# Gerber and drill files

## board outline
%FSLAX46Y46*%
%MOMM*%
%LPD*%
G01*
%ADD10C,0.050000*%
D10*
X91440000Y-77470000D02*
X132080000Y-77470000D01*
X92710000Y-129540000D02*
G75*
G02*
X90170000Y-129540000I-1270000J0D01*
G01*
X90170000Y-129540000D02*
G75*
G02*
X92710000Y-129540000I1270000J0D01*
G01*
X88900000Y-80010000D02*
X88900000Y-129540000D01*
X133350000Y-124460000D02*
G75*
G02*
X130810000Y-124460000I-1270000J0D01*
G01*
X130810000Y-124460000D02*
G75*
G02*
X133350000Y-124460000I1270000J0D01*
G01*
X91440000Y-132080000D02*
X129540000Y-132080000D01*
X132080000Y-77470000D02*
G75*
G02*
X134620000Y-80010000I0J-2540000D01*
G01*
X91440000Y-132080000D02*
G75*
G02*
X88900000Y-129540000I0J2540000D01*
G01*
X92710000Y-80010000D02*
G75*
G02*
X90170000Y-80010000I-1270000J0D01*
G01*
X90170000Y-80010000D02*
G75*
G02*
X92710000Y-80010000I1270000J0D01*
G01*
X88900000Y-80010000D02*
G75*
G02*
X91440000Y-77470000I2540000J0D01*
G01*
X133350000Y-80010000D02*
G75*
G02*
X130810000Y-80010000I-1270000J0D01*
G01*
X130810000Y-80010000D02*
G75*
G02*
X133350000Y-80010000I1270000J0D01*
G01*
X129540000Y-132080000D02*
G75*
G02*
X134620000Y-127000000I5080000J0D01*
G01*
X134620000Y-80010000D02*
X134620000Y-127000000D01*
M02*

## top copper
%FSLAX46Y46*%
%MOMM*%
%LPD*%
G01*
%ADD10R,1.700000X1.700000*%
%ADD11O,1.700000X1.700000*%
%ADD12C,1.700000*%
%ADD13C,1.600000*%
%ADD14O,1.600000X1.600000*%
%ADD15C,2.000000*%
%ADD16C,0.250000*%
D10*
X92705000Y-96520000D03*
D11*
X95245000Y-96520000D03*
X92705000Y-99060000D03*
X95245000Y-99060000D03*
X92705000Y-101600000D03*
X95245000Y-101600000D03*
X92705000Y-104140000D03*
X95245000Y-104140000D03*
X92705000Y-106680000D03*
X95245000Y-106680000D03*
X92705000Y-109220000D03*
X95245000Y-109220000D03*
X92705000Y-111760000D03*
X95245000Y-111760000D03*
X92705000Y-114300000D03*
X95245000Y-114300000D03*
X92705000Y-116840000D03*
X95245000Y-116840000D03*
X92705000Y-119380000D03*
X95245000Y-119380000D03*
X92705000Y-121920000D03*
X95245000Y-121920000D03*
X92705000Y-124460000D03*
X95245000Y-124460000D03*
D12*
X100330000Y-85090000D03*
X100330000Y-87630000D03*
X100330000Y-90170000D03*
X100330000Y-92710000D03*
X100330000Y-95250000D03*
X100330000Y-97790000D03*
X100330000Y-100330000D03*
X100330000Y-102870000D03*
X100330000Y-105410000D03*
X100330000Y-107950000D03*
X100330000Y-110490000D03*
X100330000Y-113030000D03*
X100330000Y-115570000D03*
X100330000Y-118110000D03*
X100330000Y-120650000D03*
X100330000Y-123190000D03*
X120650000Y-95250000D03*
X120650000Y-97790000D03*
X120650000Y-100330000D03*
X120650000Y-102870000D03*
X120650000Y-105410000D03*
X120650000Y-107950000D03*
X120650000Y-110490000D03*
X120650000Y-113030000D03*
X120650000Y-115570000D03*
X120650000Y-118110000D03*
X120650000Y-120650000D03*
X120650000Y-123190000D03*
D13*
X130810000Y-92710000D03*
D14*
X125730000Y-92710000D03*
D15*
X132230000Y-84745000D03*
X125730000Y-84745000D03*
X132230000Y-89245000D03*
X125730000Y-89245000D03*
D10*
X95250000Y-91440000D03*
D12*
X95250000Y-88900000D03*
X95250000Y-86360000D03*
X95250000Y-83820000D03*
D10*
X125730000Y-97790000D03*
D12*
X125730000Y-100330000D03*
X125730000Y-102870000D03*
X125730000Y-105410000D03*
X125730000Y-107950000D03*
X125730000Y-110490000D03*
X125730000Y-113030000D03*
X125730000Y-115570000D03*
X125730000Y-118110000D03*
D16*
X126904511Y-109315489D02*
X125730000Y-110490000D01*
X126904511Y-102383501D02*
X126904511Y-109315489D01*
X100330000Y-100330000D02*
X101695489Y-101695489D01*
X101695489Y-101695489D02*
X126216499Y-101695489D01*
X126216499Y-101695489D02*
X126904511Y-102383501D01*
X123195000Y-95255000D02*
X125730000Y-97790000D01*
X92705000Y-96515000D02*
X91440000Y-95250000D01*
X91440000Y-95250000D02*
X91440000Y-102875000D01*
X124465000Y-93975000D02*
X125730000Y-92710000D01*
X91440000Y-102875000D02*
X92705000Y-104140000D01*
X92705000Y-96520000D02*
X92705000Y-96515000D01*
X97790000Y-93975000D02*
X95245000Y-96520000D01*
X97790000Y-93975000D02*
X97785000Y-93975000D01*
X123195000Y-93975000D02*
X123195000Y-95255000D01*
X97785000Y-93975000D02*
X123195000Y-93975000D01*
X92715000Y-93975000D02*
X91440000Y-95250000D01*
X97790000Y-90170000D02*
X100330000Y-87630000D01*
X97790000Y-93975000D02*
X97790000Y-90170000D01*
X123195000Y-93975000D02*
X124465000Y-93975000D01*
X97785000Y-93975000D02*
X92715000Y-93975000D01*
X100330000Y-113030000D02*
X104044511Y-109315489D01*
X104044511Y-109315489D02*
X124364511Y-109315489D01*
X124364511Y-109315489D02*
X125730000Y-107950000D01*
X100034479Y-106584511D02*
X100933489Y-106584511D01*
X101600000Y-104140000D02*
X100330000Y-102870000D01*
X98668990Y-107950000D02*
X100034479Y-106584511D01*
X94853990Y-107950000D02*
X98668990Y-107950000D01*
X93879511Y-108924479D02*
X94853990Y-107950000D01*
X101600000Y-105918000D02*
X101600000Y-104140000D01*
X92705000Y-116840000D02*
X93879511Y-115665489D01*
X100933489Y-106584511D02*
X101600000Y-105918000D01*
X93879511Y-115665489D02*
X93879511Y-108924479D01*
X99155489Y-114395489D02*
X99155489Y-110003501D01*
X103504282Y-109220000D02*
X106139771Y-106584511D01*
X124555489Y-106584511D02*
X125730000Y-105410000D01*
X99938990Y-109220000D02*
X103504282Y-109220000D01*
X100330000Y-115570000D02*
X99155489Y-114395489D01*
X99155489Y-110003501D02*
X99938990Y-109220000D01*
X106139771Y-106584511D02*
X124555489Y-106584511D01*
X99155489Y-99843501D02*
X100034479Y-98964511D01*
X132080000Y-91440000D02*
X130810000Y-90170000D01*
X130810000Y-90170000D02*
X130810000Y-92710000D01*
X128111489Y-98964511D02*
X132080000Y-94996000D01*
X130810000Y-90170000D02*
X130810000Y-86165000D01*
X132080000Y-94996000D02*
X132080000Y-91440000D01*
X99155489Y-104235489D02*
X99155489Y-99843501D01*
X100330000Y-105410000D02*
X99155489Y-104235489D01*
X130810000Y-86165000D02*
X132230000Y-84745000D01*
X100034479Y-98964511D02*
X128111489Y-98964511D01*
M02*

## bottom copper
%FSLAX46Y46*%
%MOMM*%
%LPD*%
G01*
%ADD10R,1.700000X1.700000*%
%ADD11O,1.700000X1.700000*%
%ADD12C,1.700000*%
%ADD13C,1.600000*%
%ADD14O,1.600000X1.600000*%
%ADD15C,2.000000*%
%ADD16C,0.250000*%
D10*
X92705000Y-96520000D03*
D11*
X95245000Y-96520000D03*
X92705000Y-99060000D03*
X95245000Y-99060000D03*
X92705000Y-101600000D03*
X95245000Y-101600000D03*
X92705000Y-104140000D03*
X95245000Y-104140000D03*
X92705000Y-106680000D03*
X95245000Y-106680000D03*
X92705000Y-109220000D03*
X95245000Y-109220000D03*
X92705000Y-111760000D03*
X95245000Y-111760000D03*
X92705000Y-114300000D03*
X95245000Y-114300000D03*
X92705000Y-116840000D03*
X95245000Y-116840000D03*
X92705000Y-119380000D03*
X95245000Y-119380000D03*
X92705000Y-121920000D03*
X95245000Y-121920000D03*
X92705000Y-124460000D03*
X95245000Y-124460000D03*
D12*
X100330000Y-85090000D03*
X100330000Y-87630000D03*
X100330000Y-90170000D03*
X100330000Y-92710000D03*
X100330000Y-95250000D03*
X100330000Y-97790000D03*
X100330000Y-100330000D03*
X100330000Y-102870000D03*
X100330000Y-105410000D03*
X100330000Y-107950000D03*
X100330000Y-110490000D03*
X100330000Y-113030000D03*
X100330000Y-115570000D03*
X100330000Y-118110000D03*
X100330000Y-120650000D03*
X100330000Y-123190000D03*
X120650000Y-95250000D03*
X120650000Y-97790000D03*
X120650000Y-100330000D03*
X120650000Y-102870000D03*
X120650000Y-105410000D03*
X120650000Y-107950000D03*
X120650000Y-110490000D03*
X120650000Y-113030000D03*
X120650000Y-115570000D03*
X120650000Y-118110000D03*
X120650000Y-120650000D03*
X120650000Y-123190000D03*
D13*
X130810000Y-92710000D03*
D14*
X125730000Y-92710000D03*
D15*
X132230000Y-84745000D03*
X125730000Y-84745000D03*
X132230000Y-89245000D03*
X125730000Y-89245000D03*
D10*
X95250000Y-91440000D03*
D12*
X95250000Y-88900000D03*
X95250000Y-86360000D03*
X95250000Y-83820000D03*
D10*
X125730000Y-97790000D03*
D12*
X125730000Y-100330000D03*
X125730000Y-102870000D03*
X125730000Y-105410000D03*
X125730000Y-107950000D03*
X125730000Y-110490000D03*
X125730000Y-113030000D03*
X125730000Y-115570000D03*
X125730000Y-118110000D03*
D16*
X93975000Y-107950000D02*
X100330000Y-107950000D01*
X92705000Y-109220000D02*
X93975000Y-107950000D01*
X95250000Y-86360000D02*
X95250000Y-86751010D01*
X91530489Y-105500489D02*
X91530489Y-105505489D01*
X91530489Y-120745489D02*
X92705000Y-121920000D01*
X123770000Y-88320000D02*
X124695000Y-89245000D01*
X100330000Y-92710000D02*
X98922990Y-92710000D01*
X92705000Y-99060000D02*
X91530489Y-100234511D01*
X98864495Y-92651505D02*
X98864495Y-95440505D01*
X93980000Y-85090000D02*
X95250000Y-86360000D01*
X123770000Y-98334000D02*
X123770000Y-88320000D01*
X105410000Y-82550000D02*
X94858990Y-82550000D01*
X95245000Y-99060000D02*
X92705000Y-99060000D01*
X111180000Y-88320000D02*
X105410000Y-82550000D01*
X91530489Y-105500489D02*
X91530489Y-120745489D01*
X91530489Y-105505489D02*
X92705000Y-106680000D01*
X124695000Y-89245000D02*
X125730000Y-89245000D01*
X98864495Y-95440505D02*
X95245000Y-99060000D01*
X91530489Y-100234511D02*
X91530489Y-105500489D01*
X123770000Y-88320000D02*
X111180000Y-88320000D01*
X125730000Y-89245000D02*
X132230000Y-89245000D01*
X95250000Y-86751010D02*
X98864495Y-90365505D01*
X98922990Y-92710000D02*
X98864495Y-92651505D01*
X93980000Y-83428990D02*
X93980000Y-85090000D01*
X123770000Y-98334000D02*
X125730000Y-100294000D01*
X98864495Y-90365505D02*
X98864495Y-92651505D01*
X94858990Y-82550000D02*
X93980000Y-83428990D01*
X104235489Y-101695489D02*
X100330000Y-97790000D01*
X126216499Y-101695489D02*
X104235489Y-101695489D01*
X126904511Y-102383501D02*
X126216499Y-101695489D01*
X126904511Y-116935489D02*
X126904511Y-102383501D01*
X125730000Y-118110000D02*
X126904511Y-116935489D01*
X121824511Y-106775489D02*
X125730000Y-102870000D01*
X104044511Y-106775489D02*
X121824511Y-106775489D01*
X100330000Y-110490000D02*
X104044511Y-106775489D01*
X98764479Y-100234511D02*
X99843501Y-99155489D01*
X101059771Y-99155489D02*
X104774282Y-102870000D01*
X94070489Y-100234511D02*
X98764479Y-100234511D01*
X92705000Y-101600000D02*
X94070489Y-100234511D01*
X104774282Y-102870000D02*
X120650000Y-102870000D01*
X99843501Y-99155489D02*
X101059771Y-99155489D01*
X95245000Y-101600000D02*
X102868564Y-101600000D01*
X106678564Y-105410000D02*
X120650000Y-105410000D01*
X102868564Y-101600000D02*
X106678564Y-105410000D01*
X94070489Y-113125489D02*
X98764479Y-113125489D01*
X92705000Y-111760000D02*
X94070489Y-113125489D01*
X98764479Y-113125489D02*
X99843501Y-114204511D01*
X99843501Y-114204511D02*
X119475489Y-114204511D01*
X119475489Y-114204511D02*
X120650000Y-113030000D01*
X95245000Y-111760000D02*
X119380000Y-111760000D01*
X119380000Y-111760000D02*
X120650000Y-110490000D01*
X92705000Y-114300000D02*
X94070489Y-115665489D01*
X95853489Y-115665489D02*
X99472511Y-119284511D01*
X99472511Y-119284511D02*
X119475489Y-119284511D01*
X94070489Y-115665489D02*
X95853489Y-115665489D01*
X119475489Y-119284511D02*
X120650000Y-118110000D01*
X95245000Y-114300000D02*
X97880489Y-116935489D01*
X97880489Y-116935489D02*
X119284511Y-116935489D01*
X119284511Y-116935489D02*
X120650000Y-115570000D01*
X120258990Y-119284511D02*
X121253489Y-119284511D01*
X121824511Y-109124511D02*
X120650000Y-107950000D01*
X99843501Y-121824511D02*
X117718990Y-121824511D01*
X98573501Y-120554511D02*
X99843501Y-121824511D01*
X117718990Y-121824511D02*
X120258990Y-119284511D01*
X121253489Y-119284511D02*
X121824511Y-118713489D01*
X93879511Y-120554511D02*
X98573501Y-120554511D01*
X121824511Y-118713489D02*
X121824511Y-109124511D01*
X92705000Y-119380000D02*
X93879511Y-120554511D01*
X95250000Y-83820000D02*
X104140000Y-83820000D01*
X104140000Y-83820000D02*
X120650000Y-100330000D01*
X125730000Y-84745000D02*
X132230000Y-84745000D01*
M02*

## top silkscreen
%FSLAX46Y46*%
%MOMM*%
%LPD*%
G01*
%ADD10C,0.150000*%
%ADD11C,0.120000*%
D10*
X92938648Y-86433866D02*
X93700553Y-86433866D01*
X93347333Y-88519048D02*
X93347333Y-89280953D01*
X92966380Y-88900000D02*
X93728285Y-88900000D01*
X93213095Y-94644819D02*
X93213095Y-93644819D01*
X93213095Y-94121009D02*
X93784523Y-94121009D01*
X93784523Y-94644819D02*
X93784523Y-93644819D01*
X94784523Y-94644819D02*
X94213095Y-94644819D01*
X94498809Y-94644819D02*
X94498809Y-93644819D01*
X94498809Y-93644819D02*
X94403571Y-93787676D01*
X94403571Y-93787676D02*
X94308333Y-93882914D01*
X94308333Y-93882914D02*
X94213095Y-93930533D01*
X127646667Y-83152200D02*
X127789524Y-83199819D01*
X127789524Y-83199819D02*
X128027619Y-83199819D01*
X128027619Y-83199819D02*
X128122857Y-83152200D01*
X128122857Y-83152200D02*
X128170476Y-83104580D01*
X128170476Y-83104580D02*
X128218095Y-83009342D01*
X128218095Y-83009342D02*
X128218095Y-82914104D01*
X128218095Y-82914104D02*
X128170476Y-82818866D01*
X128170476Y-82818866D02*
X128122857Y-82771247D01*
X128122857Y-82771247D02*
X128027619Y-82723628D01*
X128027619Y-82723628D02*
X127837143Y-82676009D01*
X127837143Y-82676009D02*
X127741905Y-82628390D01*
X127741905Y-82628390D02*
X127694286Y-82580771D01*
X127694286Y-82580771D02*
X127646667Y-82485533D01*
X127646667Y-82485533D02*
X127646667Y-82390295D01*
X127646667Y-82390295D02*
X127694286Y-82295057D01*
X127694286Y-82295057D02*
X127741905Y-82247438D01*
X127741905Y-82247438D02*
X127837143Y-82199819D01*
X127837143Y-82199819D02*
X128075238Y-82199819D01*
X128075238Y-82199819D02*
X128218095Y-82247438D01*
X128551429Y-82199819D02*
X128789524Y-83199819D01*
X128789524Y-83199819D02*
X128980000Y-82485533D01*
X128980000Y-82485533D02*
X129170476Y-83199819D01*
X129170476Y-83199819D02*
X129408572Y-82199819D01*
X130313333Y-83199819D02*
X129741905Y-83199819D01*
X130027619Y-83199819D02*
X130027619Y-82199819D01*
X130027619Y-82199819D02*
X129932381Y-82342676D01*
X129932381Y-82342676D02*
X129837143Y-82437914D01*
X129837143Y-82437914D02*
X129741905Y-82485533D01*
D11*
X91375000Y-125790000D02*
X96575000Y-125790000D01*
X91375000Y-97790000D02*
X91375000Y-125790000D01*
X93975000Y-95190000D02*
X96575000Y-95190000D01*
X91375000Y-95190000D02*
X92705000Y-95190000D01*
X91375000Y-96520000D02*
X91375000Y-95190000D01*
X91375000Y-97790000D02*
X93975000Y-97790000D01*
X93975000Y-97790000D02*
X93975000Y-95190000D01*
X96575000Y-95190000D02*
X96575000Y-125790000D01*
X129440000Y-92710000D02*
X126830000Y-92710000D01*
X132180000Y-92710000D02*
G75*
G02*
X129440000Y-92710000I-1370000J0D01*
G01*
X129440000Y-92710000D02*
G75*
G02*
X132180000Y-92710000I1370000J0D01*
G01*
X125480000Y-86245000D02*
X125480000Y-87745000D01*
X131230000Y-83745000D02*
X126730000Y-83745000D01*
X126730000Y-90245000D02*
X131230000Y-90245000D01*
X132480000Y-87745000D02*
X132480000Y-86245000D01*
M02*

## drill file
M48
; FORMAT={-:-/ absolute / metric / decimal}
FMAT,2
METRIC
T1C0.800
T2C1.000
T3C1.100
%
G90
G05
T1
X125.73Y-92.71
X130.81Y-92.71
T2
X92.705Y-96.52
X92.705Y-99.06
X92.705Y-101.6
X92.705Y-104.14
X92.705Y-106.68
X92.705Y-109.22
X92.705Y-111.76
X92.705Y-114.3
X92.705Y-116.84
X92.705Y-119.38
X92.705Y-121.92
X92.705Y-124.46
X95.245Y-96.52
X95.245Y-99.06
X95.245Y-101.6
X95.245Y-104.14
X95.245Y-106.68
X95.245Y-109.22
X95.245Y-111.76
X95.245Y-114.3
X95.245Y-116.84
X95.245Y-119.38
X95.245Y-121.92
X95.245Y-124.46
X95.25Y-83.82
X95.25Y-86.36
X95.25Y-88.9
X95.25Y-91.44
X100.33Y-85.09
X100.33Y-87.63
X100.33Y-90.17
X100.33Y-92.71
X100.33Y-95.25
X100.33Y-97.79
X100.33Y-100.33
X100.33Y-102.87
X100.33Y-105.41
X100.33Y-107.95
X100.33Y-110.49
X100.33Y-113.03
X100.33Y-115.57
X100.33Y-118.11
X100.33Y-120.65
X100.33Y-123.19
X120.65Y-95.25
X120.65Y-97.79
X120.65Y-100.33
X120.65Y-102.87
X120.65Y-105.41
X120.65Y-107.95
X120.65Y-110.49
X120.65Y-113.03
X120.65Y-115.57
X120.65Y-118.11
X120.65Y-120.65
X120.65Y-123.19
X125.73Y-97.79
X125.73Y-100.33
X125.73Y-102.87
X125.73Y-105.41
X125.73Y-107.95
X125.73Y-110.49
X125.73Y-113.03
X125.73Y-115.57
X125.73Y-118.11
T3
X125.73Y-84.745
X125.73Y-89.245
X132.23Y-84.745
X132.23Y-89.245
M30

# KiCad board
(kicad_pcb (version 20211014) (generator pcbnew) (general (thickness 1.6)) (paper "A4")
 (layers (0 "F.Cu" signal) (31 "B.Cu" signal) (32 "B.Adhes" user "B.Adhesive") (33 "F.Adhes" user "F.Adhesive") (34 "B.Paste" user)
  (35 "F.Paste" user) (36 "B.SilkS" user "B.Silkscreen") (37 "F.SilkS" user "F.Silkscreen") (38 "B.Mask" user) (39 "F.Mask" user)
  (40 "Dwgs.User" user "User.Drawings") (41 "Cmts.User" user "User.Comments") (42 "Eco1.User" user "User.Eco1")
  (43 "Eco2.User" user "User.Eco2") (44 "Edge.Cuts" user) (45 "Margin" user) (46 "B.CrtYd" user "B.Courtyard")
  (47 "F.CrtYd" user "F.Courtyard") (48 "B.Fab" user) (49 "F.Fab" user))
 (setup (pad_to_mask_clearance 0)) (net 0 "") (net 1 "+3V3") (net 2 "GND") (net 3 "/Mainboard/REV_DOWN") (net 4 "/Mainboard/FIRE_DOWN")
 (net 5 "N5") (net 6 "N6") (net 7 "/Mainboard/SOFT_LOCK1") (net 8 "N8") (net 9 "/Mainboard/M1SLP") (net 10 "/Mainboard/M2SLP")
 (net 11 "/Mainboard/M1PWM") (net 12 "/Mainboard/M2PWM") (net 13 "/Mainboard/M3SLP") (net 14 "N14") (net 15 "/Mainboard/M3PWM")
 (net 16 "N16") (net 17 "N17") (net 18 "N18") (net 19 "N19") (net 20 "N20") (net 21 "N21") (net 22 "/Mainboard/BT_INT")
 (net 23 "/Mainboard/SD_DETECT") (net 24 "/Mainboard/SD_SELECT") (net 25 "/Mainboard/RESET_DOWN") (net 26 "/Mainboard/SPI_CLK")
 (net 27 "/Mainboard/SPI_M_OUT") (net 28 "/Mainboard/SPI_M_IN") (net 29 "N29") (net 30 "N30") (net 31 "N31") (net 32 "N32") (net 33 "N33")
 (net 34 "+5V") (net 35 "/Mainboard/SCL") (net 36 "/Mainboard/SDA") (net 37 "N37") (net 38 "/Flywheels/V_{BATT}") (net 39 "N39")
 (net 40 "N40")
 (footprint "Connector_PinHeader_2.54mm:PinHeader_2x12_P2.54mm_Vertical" (layer "F.Cu") (at 92.705 96.52)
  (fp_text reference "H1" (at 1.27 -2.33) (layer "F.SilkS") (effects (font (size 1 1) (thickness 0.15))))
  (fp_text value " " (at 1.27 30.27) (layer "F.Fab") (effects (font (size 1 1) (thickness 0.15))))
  (fp_line (start -1.33 29.27) (end 3.87 29.27) (layer "F.SilkS") (width 0.12))
  (fp_line (start -1.33 1.27) (end -1.33 29.27) (layer "F.SilkS") (width 0.12))
  (fp_line (start 1.27 -1.33) (end 3.87 -1.33) (layer "F.SilkS") (width 0.12))
  (fp_line (start -1.33 -1.33) (end 0 -1.33) (layer "F.SilkS") (width 0.12))
  (fp_line (start -1.33 0) (end -1.33 -1.33) (layer "F.SilkS") (width 0.12))
  (fp_line (start -1.33 1.27) (end 1.27 1.27) (layer "F.SilkS") (width 0.12))
  (fp_line (start 1.27 1.27) (end 1.27 -1.33) (layer "F.SilkS") (width 0.12))
  (fp_line (start 3.87 -1.33) (end 3.87 29.27) (layer "F.SilkS") (width 0.12))
  (pad "1" thru_hole rect locked (at 0 0) (size 1.7 1.7) (drill 1) (layers *.Cu *.Mask) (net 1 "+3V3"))
  (pad "2" thru_hole oval locked (at 2.54 0) (size 1.7 1.7) (drill 1) (layers *.Cu *.Mask) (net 1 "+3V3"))
  (pad "3" thru_hole oval locked (at 0 2.54) (size 1.7 1.7) (drill 1) (layers *.Cu *.Mask) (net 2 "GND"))
  (pad "4" thru_hole oval locked (at 2.54 2.54) (size 1.7 1.7) (drill 1) (layers *.Cu *.Mask) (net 2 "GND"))
  (pad "5" thru_hole oval locked (at 0 5.08) (size 1.7 1.7) (drill 1) (layers *.Cu *.Mask) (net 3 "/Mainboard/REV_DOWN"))
  (pad "6" thru_hole oval locked (at 2.54 5.08) (size 1.7 1.7) (drill 1) (layers *.Cu *.Mask) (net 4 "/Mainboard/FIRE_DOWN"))
  (pad "7" thru_hole oval locked (at 0 7.62) (size 1.7 1.7) (drill 1) (layers *.Cu *.Mask) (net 1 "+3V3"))
  (pad "8" thru_hole oval locked (at 2.54 7.62) (size 1.7 1.7) (drill 1) (layers *.Cu *.Mask) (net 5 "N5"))
  (pad "9" thru_hole oval locked (at 0 10.16) (size 1.7 1.7) (drill 1) (layers *.Cu *.Mask) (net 2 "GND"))
  (pad "10" thru_hole oval locked (at 2.54 10.16) (size 1.7 1.7) (drill 1) (layers *.Cu *.Mask) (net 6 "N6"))
  (pad "11" thru_hole oval locked (at 0 12.7) (size 1.7 1.7) (drill 1) (layers *.Cu *.Mask) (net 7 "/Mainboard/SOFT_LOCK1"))
  (pad "12" thru_hole oval locked (at 2.54 12.7) (size 1.7 1.7) (drill 1) (layers *.Cu *.Mask) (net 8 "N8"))
  (pad "13" thru_hole oval locked (at 0 15.24) (size 1.7 1.7) (drill 1) (layers *.Cu *.Mask) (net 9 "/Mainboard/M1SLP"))
  (pad "14" thru_hole oval locked (at 2.54 15.24) (size 1.7 1.7) (drill 1) (layers *.Cu *.Mask) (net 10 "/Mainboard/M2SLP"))
  (pad "15" thru_hole oval locked (at 0 17.78) (size 1.7 1.7) (drill 1) (layers *.Cu *.Mask) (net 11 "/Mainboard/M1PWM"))
  (pad "16" thru_hole oval locked (at 2.54 17.78) (size 1.7 1.7) (drill 1) (layers *.Cu *.Mask) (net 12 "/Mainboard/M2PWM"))
  (pad "17" thru_hole oval locked (at 0 20.32) (size 1.7 1.7) (drill 1) (layers *.Cu *.Mask) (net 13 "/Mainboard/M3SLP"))
  (pad "18" thru_hole oval locked (at 2.54 20.32) (size 1.7 1.7) (drill 1) (layers *.Cu *.Mask) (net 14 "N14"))
  (pad "19" thru_hole oval locked (at 0 22.86) (size 1.7 1.7) (drill 1) (layers *.Cu *.Mask) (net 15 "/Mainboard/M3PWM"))
  (pad "20" thru_hole oval locked (at 2.54 22.86) (size 1.7 1.7) (drill 1) (layers *.Cu *.Mask) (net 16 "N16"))
  (pad "21" thru_hole oval locked (at 0 25.4) (size 1.7 1.7) (drill 1) (layers *.Cu *.Mask) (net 2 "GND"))
  (pad "22" thru_hole oval locked (at 2.54 25.4) (size 1.7 1.7) (drill 1) (layers *.Cu *.Mask) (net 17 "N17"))
  (pad "23" thru_hole oval locked (at 0 27.94) (size 1.7 1.7) (drill 1) (layers *.Cu *.Mask) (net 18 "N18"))
  (pad "24" thru_hole oval locked (at 2.54 27.94) (size 1.7 1.7) (drill 1) (layers *.Cu *.Mask) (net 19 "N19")))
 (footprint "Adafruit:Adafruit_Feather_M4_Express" (layer "F.Cu") (at 110.49 104.14)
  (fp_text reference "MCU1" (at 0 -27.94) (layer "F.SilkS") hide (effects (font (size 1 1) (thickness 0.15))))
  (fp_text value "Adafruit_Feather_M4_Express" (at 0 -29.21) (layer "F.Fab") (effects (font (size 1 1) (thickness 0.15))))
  (pad "1" thru_hole circle (at -10.16 -19.05) (size 1.7 1.7) (drill 1) (layers *.Cu *.Mask) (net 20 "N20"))
  (pad "2" thru_hole circle (at -10.16 -16.51) (size 1.7 1.7) (drill 1) (layers *.Cu *.Mask) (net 1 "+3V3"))
  (pad "3" thru_hole circle (at -10.16 -13.97) (size 1.7 1.7) (drill 1) (layers *.Cu *.Mask) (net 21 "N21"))
  (pad "4" thru_hole circle (at -10.16 -11.43) (size 1.7 1.7) (drill 1) (layers *.Cu *.Mask) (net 2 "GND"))
  (pad "5" thru_hole circle (at -10.16 -8.89) (size 1.7 1.7) (drill 1) (layers *.Cu *.Mask) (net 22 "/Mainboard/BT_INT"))
  (pad "6" thru_hole circle (at -10.16 -6.35) (size 1.7 1.7) (drill 1) (layers *.Cu *.Mask) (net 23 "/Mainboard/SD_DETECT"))
  (pad "7" thru_hole circle (at -10.16 -3.81) (size 1.7 1.7) (drill 1) (layers *.Cu *.Mask) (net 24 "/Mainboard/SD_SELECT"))
  (pad "8" thru_hole circle (at -10.16 -1.27) (size 1.7 1.7) (drill 1) (layers *.Cu *.Mask) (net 13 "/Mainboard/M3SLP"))
  (pad "9" thru_hole circle (at -10.16 1.27) (size 1.7 1.7) (drill 1) (layers *.Cu *.Mask) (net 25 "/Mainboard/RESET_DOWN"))
  (pad "10" thru_hole circle (at -10.16 3.81) (size 1.7 1.7) (drill 1) (layers *.Cu *.Mask) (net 7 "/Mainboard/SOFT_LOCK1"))
  (pad "11" thru_hole circle (at -10.16 6.35) (size 1.7 1.7) (drill 1) (layers *.Cu *.Mask) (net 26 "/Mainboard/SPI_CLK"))
  (pad "12" thru_hole circle (at -10.16 8.89) (size 1.7 1.7) (drill 1) (layers *.Cu *.Mask) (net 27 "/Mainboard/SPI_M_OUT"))
  (pad "13" thru_hole circle (at -10.16 11.43) (size 1.7 1.7) (drill 1) (layers *.Cu *.Mask) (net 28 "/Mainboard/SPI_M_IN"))
  (pad "14" thru_hole circle (at -10.16 13.97) (size 1.7 1.7) (drill 1) (layers *.Cu *.Mask) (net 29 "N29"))
  (pad "15" thru_hole circle (at -10.16 16.51) (size 1.7 1.7) (drill 1) (layers *.Cu *.Mask) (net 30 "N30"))
  (pad "16" thru_hole circle (at -10.16 19.05) (size 1.7 1.7) (drill 1) (layers *.Cu *.Mask) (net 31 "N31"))
  (pad "17" thru_hole circle (at 10.16 -8.89) (size 1.7 1.7) (drill 1) (layers *.Cu *.Mask) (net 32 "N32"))
  (pad "18" thru_hole circle (at 10.16 -6.35) (size 1.7 1.7) (drill 1) (layers *.Cu *.Mask) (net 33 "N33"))
  (pad "19" thru_hole circle (at 10.16 -3.81) (size 1.7 1.7) (drill 1) (layers *.Cu *.Mask) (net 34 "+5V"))
  (pad "20" thru_hole circle (at 10.16 -1.27) (size 1.7 1.7) (drill 1) (layers *.Cu *.Mask) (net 3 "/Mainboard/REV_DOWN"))
  (pad "21" thru_hole circle (at 10.16 1.27) (size 1.7 1.7) (drill 1) (layers *.Cu *.Mask) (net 4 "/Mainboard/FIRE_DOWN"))
  (pad "22" thru_hole circle (at 10.16 3.81) (size 1.7 1.7) (drill 1) (layers *.Cu *.Mask) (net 15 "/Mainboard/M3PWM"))
  (pad "23" thru_hole circle (at 10.16 6.35) (size 1.7 1.7) (drill 1) (layers *.Cu *.Mask) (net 10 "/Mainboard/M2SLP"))
  (pad "24" thru_hole circle (at 10.16 8.89) (size 1.7 1.7) (drill 1) (layers *.Cu *.Mask) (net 9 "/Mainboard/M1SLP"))
  (pad "25" thru_hole circle (at 10.16 11.43) (size 1.7 1.7) (drill 1) (layers *.Cu *.Mask) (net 12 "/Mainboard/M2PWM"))
  (pad "26" thru_hole circle (at 10.16 13.97) (size 1.7 1.7) (drill 1) (layers *.Cu *.Mask) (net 11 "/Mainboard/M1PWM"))
  (pad "27" thru_hole circle (at 10.16 16.51) (size 1.7 1.7) (drill 1) (layers *.Cu *.Mask) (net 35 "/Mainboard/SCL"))
  (pad "28" thru_hole circle (at 10.16 19.05) (size 1.7 1.7) (drill 1) (layers *.Cu *.Mask) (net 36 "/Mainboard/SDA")))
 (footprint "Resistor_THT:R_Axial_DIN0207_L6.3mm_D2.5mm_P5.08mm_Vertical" (layer "F.Cu") (at 130.81 92.71 180)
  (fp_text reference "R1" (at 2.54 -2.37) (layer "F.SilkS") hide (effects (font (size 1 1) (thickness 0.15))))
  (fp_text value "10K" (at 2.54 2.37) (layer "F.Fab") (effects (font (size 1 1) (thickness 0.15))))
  (fp_line (start 1.37 0) (end 3.98 0) (layer "F.SilkS") (width 0.12))
  (fp_circle (center 0 0) (end 1.37 0) (layer "F.SilkS") (width 0.12) (fill none))
  (pad "1" thru_hole circle locked (at 0 0 180) (size 1.6 1.6) (drill 0.8) (layers *.Cu *.Mask) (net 25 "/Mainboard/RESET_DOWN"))
  (pad "2" thru_hole oval locked (at 5.08 0 180) (size 1.6 1.6) (drill 0.8) (layers *.Cu *.Mask) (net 1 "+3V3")))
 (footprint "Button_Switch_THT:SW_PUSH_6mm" (layer "F.Cu") (at 125.73 84.745)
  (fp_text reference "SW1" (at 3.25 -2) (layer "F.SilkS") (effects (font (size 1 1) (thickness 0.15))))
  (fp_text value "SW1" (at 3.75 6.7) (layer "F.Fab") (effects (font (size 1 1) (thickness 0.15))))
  (fp_line (start -0.25 1.5) (end -0.25 3) (layer "F.SilkS") (width 0.12))
  (fp_line (start 5.5 -1) (end 1 -1) (layer "F.SilkS") (width 0.12))
  (fp_line (start 1 5.5) (end 5.5 5.5) (layer "F.SilkS") (width 0.12))
  (fp_line (start 6.75 3) (end 6.75 1.5) (layer "F.SilkS") (width 0.12))
  (pad "1" thru_hole circle locked (at 6.5 0 90) (size 2 2) (drill 1.1) (layers *.Cu *.Mask) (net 25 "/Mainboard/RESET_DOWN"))
  (pad "1" thru_hole circle locked (at 0 0 90) (size 2 2) (drill 1.1) (layers *.Cu *.Mask) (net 25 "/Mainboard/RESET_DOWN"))
  (pad "2" thru_hole circle locked (at 6.5 4.5 90) (size 2 2) (drill 1.1) (layers *.Cu *.Mask) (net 2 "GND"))
  (pad "2" thru_hole circle locked (at 0 4.5 90) (size 2 2) (drill 1.1) (layers *.Cu *.Mask) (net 2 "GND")))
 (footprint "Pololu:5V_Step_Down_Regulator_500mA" (layer "B.Cu") (at 100.33 87.63 90)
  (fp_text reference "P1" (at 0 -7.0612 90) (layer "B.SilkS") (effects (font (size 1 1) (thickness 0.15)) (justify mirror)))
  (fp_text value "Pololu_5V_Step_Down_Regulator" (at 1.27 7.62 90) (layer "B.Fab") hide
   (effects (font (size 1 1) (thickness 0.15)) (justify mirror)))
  (pad "1" thru_hole rect (at -3.81 -5.08 90) (size 1.7 1.7) (drill 1) (layers *.Cu *.Mask) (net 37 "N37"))
  (pad "2" thru_hole circle (at -1.27 -5.08 90) (size 1.7 1.7) (drill 1) (layers *.Cu *.Mask) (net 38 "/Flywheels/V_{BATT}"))
  (pad "3" thru_hole circle (at 1.27 -5.08 90) (size 1.7 1.7) (drill 1) (layers *.Cu *.Mask) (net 2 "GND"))
  (pad "4" thru_hole circle (at 3.81 -5.08 90) (size 1.7 1.7) (drill 1) (layers *.Cu *.Mask) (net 34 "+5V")))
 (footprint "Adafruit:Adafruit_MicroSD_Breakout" (layer "B.Cu") (at 116.84 108.712 -90)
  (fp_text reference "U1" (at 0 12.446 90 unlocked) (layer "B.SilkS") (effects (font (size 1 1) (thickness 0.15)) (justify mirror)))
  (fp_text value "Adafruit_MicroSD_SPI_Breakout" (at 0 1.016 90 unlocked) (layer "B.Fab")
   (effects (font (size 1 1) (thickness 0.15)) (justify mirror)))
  (pad "1" thru_hole rect (at -10.922 -8.89 270) (size 1.7 1.7) (drill 1) (layers *.Cu *.Mask) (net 1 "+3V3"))
  (pad "2" thru_hole circle (at -8.382 -8.89 270) (size 1.7 1.7) (drill 1) (layers *.Cu *.Mask) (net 2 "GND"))
  (pad "3" thru_hole circle (at -5.842 -8.89 270) (size 1.7 1.7) (drill 1) (layers *.Cu *.Mask) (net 26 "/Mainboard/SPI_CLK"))
  (pad "4" thru_hole circle (at -3.302 -8.89 270) (size 1.7 1.7) (drill 1) (layers *.Cu *.Mask) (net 28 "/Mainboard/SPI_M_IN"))
  (pad "5" thru_hole circle (at -0.762 -8.89 270) (size 1.7 1.7) (drill 1) (layers *.Cu *.Mask) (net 27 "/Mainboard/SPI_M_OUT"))
  (pad "6" thru_hole circle (at 1.778 -8.89 270) (size 1.7 1.7) (drill 1) (layers *.Cu *.Mask) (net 24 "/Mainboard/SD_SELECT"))
  (pad "7" thru_hole circle (at 4.318 -8.89 270) (size 1.7 1.7) (drill 1) (layers *.Cu *.Mask) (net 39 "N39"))
  (pad "8" thru_hole circle (at 6.858 -8.89 270) (size 1.7 1.7) (drill 1) (layers *.Cu *.Mask) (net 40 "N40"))
  (pad "9" thru_hole circle (at 9.398 -8.89 270) (size 1.7 1.7) (drill 1) (layers *.Cu *.Mask) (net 23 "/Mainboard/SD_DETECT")))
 (gr_line (start 91.44 77.47) (end 132.08 77.47) (layer "Edge.Cuts") (width 0.05))
 (gr_circle (center 91.44 129.54) (end 91.44 130.81) (layer "Edge.Cuts") (width 0.05) (fill none))
 (gr_line (start 88.9 80.01) (end 88.9 129.54) (layer "Edge.Cuts") (width 0.05))
 (gr_circle (center 132.08 124.46) (end 133.35 124.46) (layer "Edge.Cuts") (width 0.05) (fill none))
 (gr_line (start 91.44 132.08) (end 129.54 132.08) (layer "Edge.Cuts") (width 0.05))
 (gr_arc (start 132.08 77.47) (mid 133.876051 78.213949) (end 134.62 80.01) (layer "Edge.Cuts") (width 0.05))
 (gr_arc (start 91.44 132.08) (mid 89.643949 131.336051) (end 88.9 129.54) (layer "Edge.Cuts") (width 0.05))
 (gr_circle (center 91.44 80.01) (end 90.17 80.01) (layer "Edge.Cuts") (width 0.05) (fill none))
 (gr_arc (start 88.9 80.01) (mid 89.643949 78.213949) (end 91.44 77.47) (layer "Edge.Cuts") (width 0.05))
 (gr_circle (center 132.08 80.01) (end 133.35 80.01) (layer "Edge.Cuts") (width 0.05) (fill none))
 (gr_arc (start 129.54 132.08) (mid 131.027898 128.487898) (end 134.62 127) (layer "Edge.Cuts") (width 0.05))
 (gr_line (start 134.62 80.01) (end 134.62 127) (layer "Edge.Cuts") (width 0.05))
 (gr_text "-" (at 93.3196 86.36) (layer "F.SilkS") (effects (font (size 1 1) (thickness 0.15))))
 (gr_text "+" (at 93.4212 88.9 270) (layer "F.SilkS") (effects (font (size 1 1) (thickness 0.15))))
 (segment (start 93.975 107.95) (end 100.33 107.95) (width 0.25) (layer "B.Cu") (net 7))
 (segment (start 92.705 109.22) (end 93.975 107.95) (width 0.25) (layer "B.Cu") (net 7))
 (segment (start 95.25 86.36) (end 95.25 86.75101) (width 0.25) (layer "B.Cu") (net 2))
 (segment (start 91.530489 105.500489) (end 91.530489 105.505489) (width 0.25) (layer "B.Cu") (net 2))
 (segment (start 91.530489 120.745489) (end 92.705 121.92) (width 0.25) (layer "B.Cu") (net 2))
 (segment (start 123.77 88.32) (end 124.695 89.245) (width 0.25) (layer "B.Cu") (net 2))
 (segment (start 100.33 92.71) (end 98.92299 92.71) (width 0.25) (layer "B.Cu") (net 2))
 (segment (start 92.705 99.06) (end 91.530489 100.234511) (width 0.25) (layer "B.Cu") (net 2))
 (segment (start 98.864495 92.651505) (end 98.864495 95.440505) (width 0.25) (layer "B.Cu") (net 2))
 (segment (start 93.98 85.09) (end 95.25 86.36) (width 0.25) (layer "B.Cu") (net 2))
 (segment (start 123.77 98.334) (end 123.77 88.32) (width 0.25) (layer "B.Cu") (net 2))
 (segment (start 105.41 82.55) (end 94.85899 82.55) (width 0.25) (layer "B.Cu") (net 2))
 (segment (start 95.245 99.06) (end 92.705 99.06) (width 0.25) (layer "B.Cu") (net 2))
 (segment (start 111.18 88.32) (end 105.41 82.55) (width 0.25) (layer "B.Cu") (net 2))
 (segment (start 91.530489 105.500489) (end 91.530489 120.745489) (width 0.25) (layer "B.Cu") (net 2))
 (segment (start 91.530489 105.505489) (end 92.705 106.68) (width 0.25) (layer "B.Cu") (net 2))
 (segment (start 124.695 89.245) (end 125.73 89.245) (width 0.25) (layer "B.Cu") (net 2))
 (segment (start 98.864495 95.440505) (end 95.245 99.06) (width 0.25) (layer "B.Cu") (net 2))
 (segment (start 91.530489 100.234511) (end 91.530489 105.500489) (width 0.25) (layer "B.Cu") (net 2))
 (segment (start 123.77 88.32) (end 111.18 88.32) (width 0.25) (layer "B.Cu") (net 2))
 (segment (start 125.73 89.245) (end 132.23 89.245) (width 0.25) (layer "B.Cu") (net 2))
 (segment (start 95.25 86.75101) (end 98.864495 90.365505) (width 0.25) (layer "B.Cu") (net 2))
 (segment (start 98.92299 92.71) (end 98.864495 92.651505) (width 0.25) (layer "B.Cu") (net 2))
 (segment (start 93.98 83.42899) (end 93.98 85.09) (width 0.25) (layer "B.Cu") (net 2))
 (segment (start 123.77 98.334) (end 125.73 100.294) (width 0.25) (layer "B.Cu") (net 2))
 (segment (start 98.864495 90.365505) (end 98.864495 92.651505) (width 0.25) (layer "B.Cu") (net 2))
 (segment (start 94.85899 82.55) (end 93.98 83.42899) (width 0.25) (layer "B.Cu") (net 2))
 (segment (start 104.235489 101.695489) (end 100.33 97.79) (width 0.25) (layer "B.Cu") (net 23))
 (segment (start 126.216499 101.695489) (end 104.235489 101.695489) (width 0.25) (layer "B.Cu") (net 23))
 (segment (start 126.904511 102.383501) (end 126.216499 101.695489) (width 0.25) (layer "B.Cu") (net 23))
 (segment (start 126.904511 116.935489) (end 126.904511 102.383501) (width 0.25) (layer "B.Cu") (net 23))
 (segment (start 125.73 118.11) (end 126.904511 116.935489) (width 0.25) (layer "B.Cu") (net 23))
 (segment (start 126.904511 109.315489) (end 125.73 110.49) (width 0.25) (layer "F.Cu") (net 24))
 (segment (start 126.904511 102.383501) (end 126.904511 109.315489) (width 0.25) (layer "F.Cu") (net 24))
 (segment (start 100.33 100.33) (end 101.695489 101.695489) (width 0.25) (layer "F.Cu") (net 24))
 (segment (start 101.695489 101.695489) (end 126.216499 101.695489) (width 0.25) (layer "F.Cu") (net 24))
 (segment (start 126.216499 101.695489) (end 126.904511 102.383501) (width 0.25) (layer "F.Cu") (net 24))
 (segment (start 121.824511 106.775489) (end 125.73 102.87) (width 0.25) (layer "B.Cu") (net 26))
 (segment (start 104.044511 106.775489) (end 121.824511 106.775489) (width 0.25) (layer "B.Cu") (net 26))
 (segment (start 100.33 110.49) (end 104.044511 106.775489) (width 0.25) (layer "B.Cu") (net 26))
 (segment (start 123.195 95.255) (end 125.73 97.79) (width 0.25) (layer "F.Cu") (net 1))
 (segment (start 92.705 96.515) (end 91.44 95.25) (width 0.25) (layer "F.Cu") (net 1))
 (segment (start 91.44 95.25) (end 91.44 102.875) (width 0.25) (layer "F.Cu") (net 1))
 (segment (start 124.465 93.975) (end 125.73 92.71) (width 0.25) (layer "F.Cu") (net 1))
 (segment (start 91.44 102.875) (end 92.705 104.14) (width 0.25) (layer "F.Cu") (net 1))
 (segment (start 92.705 96.52) (end 92.705 96.515) (width 0.25) (layer "F.Cu") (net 1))
 (segment (start 97.79 93.975) (end 95.245 96.52) (width 0.25) (layer "F.Cu") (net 1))
 (segment (start 97.79 93.975) (end 97.785 93.975) (width 0.25) (layer "F.Cu") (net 1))
 (segment (start 123.195 93.975) (end 123.195 95.255) (width 0.25) (layer "F.Cu") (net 1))
 (segment (start 97.785 93.975) (end 123.195 93.975) (width 0.25) (layer "F.Cu") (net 1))
 (segment (start 92.715 93.975) (end 91.44 95.25) (width 0.25) (layer "F.Cu") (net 1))
 (segment (start 97.79 90.17) (end 100.33 87.63) (width 0.25) (layer "F.Cu") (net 1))
 (segment (start 97.79 93.975) (end 97.79 90.17) (width 0.25) (layer "F.Cu") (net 1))
 (segment (start 123.195 93.975) (end 124.465 93.975) (width 0.25) (layer "F.Cu") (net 1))
 (segment (start 97.785 93.975) (end 92.715 93.975) (width 0.25) (layer "F.Cu") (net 1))
 (segment (start 98.764479 100.234511) (end 99.843501 99.155489) (width 0.25) (layer "B.Cu") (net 3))
 (segment (start 101.059771 99.155489) (end 104.774282 102.87) (width 0.25) (layer "B.Cu") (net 3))
 (segment (start 94.070489 100.234511) (end 98.764479 100.234511) (width 0.25) (layer "B.Cu") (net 3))
 (segment (start 92.705 101.6) (end 94.070489 100.234511) (width 0.25) (layer "B.Cu") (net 3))
 (segment (start 104.774282 102.87) (end 120.65 102.87) (width 0.25) (layer "B.Cu") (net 3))
 (segment (start 99.843501 99.155489) (end 101.059771 99.155489) (width 0.25) (layer "B.Cu") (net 3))
 (segment (start 95.245 101.6) (end 102.868564 101.6) (width 0.25) (layer "B.Cu") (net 4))
 (segment (start 106.678564 105.41) (end 120.65 105.41) (width 0.25) (layer "B.Cu") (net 4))
 (segment (start 102.868564 101.6) (end 106.678564 105.41) (width 0.25) (layer "B.Cu") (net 4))
 (segment (start 100.33 113.03) (end 104.044511 109.315489) (width 0.25) (layer "F.Cu") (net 27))
 (segment (start 104.044511 109.315489) (end 124.364511 109.315489) (width 0.25) (layer "F.Cu") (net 27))
 (segment (start 124.364511 109.315489) (end 125.73 107.95) (width 0.25) (layer "F.Cu") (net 27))
 (segment (start 94.070489 113.125489) (end 98.764479 113.125489) (width 0.25) (layer "B.Cu") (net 9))
 (segment (start 92.705 111.76) (end 94.070489 113.125489) (width 0.25) (layer "B.Cu") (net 9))
 (segment (start 98.764479 113.125489) (end 99.843501 114.204511) (width 0.25) (layer "B.Cu") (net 9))
 (segment (start 99.843501 114.204511) (end 119.475489 114.204511) (width 0.25) (layer "B.Cu") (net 9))
 (segment (start 119.475489 114.204511) (end 120.65 113.03) (width 0.25) (layer "B.Cu") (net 9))
 (segment (start 95.245 111.76) (end 119.38 111.76) (width 0.25) (layer "B.Cu") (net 10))
 (segment (start 119.38 111.76) (end 120.65 110.49) (width 0.25) (layer "B.Cu") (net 10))
 (segment (start 92.705 114.3) (end 94.070489 115.665489) (width 0.25) (layer "B.Cu") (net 11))
 (segment (start 95.853489 115.665489) (end 99.472511 119.284511) (width 0.25) (layer "B.Cu") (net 11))
 (segment (start 99.472511 119.284511) (end 119.475489 119.284511) (width 0.25) (layer "B.Cu") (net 11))
 (segment (start 94.070489 115.665489) (end 95.853489 115.665489) (width 0.25) (layer "B.Cu") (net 11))
 (segment (start 119.475489 119.284511) (end 120.65 118.11) (width 0.25) (layer "B.Cu") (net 11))
 (segment (start 95.245 114.3) (end 97.880489 116.935489) (width 0.25) (layer "B.Cu") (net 12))
 (segment (start 97.880489 116.935489) (end 119.284511 116.935489) (width 0.25) (layer "B.Cu") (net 12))
 (segment (start 119.284511 116.935489) (end 120.65 115.57) (width 0.25) (layer "B.Cu") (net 12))
 (segment (start 100.034479 106.584511) (end 100.933489 106.584511) (width 0.25) (layer "F.Cu") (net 13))
 (segment (start 101.6 104.14) (end 100.33 102.87) (width 0.25) (layer "F.Cu") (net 13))
 (segment (start 98.66899 107.95) (end 100.034479 106.584511) (width 0.25) (layer "F.Cu") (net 13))
 (segment (start 94.85399 107.95) (end 98.66899 107.95) (width 0.25) (layer "F.Cu") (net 13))
 (segment (start 93.879511 108.924479) (end 94.85399 107.95) (width 0.25) (layer "F.Cu") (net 13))
 (segment (start 101.6 105.918) (end 101.6 104.14) (width 0.25) (layer "F.Cu") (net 13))
 (segment (start 92.705 116.84) (end 93.879511 115.665489) (width 0.25) (layer "F.Cu") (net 13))
 (segment (start 100.933489 106.584511) (end 101.6 105.918) (width 0.25) (layer "F.Cu") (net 13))
 (segment (start 93.879511 115.665489) (end 93.879511 108.924479) (width 0.25) (layer "F.Cu") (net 13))
 (segment (start 120.25899 119.284511) (end 121.253489 119.284511) (width 0.25) (layer "B.Cu") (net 15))
 (segment (start 121.824511 109.124511) (end 120.65 107.95) (width 0.25) (layer "B.Cu") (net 15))
 (segment (start 99.843501 121.824511) (end 117.71899 121.824511) (width 0.25) (layer "B.Cu") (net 15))
 (segment (start 98.573501 120.554511) (end 99.843501 121.824511) (width 0.25) (layer "B.Cu") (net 15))
 (segment (start 117.71899 121.824511) (end 120.25899 119.284511) (width 0.25) (layer "B.Cu") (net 15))
 (segment (start 121.253489 119.284511) (end 121.824511 118.713489) (width 0.25) (layer "B.Cu") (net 15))
 (segment (start 93.879511 120.554511) (end 98.573501 120.554511) (width 0.25) (layer "B.Cu") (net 15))
 (segment (start 121.824511 118.713489) (end 121.824511 109.124511) (width 0.25) (layer "B.Cu") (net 15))
 (segment (start 92.705 119.38) (end 93.879511 120.554511) (width 0.25) (layer "B.Cu") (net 15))
 (segment (start 95.25 83.82) (end 104.14 83.82) (width 0.25) (layer "B.Cu") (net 34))
 (segment (start 104.14 83.82) (end 120.65 100.33) (width 0.25) (layer "B.Cu") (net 34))
 (segment (start 99.155489 114.395489) (end 99.155489 110.003501) (width 0.25) (layer "F.Cu") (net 28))
 (segment (start 103.504282 109.22) (end 106.139771 106.584511) (width 0.25) (layer "F.Cu") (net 28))
 (segment (start 124.555489 106.584511) (end 125.73 105.41) (width 0.25) (layer "F.Cu") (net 28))
 (segment (start 99.93899 109.22) (end 103.504282 109.22) (width 0.25) (layer "F.Cu") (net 28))
 (segment (start 100.33 115.57) (end 99.155489 114.395489) (width 0.25) (layer "F.Cu") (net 28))
 (segment (start 99.155489 110.003501) (end 99.93899 109.22) (width 0.25) (layer "F.Cu") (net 28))
 (segment (start 106.139771 106.584511) (end 124.555489 106.584511) (width 0.25) (layer "F.Cu") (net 28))
 (segment (start 99.155489 99.843501) (end 100.034479 98.964511) (width 0.25) (layer "F.Cu") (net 25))
 (segment (start 132.08 91.44) (end 130.81 90.17) (width 0.25) (layer "F.Cu") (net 25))
 (segment (start 130.81 90.17) (end 130.81 92.71) (width 0.25) (layer "F.Cu") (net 25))
 (segment (start 128.111489 98.964511) (end 132.08 94.996) (width 0.25) (layer "F.Cu") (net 25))
 (segment (start 130.81 90.17) (end 130.81 86.165) (width 0.25) (layer "F.Cu") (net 25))
 (segment (start 132.08 94.996) (end 132.08 91.44) (width 0.25) (layer "F.Cu") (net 25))
 (segment (start 99.155489 104.235489) (end 99.155489 99.843501) (width 0.25) (layer "F.Cu") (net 25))
 (segment (start 100.33 105.41) (end 99.155489 104.235489) (width 0.25) (layer "F.Cu") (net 25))
 (segment (start 130.81 86.165) (end 132.23 84.745) (width 0.25) (layer "F.Cu") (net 25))
 (segment (start 100.034479 98.964511) (end 128.111489 98.964511) (width 0.25) (layer "F.Cu") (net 25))
 (segment (start 125.73 84.745) (end 132.23 84.745) (width 0.25) (layer "B.Cu") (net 25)))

